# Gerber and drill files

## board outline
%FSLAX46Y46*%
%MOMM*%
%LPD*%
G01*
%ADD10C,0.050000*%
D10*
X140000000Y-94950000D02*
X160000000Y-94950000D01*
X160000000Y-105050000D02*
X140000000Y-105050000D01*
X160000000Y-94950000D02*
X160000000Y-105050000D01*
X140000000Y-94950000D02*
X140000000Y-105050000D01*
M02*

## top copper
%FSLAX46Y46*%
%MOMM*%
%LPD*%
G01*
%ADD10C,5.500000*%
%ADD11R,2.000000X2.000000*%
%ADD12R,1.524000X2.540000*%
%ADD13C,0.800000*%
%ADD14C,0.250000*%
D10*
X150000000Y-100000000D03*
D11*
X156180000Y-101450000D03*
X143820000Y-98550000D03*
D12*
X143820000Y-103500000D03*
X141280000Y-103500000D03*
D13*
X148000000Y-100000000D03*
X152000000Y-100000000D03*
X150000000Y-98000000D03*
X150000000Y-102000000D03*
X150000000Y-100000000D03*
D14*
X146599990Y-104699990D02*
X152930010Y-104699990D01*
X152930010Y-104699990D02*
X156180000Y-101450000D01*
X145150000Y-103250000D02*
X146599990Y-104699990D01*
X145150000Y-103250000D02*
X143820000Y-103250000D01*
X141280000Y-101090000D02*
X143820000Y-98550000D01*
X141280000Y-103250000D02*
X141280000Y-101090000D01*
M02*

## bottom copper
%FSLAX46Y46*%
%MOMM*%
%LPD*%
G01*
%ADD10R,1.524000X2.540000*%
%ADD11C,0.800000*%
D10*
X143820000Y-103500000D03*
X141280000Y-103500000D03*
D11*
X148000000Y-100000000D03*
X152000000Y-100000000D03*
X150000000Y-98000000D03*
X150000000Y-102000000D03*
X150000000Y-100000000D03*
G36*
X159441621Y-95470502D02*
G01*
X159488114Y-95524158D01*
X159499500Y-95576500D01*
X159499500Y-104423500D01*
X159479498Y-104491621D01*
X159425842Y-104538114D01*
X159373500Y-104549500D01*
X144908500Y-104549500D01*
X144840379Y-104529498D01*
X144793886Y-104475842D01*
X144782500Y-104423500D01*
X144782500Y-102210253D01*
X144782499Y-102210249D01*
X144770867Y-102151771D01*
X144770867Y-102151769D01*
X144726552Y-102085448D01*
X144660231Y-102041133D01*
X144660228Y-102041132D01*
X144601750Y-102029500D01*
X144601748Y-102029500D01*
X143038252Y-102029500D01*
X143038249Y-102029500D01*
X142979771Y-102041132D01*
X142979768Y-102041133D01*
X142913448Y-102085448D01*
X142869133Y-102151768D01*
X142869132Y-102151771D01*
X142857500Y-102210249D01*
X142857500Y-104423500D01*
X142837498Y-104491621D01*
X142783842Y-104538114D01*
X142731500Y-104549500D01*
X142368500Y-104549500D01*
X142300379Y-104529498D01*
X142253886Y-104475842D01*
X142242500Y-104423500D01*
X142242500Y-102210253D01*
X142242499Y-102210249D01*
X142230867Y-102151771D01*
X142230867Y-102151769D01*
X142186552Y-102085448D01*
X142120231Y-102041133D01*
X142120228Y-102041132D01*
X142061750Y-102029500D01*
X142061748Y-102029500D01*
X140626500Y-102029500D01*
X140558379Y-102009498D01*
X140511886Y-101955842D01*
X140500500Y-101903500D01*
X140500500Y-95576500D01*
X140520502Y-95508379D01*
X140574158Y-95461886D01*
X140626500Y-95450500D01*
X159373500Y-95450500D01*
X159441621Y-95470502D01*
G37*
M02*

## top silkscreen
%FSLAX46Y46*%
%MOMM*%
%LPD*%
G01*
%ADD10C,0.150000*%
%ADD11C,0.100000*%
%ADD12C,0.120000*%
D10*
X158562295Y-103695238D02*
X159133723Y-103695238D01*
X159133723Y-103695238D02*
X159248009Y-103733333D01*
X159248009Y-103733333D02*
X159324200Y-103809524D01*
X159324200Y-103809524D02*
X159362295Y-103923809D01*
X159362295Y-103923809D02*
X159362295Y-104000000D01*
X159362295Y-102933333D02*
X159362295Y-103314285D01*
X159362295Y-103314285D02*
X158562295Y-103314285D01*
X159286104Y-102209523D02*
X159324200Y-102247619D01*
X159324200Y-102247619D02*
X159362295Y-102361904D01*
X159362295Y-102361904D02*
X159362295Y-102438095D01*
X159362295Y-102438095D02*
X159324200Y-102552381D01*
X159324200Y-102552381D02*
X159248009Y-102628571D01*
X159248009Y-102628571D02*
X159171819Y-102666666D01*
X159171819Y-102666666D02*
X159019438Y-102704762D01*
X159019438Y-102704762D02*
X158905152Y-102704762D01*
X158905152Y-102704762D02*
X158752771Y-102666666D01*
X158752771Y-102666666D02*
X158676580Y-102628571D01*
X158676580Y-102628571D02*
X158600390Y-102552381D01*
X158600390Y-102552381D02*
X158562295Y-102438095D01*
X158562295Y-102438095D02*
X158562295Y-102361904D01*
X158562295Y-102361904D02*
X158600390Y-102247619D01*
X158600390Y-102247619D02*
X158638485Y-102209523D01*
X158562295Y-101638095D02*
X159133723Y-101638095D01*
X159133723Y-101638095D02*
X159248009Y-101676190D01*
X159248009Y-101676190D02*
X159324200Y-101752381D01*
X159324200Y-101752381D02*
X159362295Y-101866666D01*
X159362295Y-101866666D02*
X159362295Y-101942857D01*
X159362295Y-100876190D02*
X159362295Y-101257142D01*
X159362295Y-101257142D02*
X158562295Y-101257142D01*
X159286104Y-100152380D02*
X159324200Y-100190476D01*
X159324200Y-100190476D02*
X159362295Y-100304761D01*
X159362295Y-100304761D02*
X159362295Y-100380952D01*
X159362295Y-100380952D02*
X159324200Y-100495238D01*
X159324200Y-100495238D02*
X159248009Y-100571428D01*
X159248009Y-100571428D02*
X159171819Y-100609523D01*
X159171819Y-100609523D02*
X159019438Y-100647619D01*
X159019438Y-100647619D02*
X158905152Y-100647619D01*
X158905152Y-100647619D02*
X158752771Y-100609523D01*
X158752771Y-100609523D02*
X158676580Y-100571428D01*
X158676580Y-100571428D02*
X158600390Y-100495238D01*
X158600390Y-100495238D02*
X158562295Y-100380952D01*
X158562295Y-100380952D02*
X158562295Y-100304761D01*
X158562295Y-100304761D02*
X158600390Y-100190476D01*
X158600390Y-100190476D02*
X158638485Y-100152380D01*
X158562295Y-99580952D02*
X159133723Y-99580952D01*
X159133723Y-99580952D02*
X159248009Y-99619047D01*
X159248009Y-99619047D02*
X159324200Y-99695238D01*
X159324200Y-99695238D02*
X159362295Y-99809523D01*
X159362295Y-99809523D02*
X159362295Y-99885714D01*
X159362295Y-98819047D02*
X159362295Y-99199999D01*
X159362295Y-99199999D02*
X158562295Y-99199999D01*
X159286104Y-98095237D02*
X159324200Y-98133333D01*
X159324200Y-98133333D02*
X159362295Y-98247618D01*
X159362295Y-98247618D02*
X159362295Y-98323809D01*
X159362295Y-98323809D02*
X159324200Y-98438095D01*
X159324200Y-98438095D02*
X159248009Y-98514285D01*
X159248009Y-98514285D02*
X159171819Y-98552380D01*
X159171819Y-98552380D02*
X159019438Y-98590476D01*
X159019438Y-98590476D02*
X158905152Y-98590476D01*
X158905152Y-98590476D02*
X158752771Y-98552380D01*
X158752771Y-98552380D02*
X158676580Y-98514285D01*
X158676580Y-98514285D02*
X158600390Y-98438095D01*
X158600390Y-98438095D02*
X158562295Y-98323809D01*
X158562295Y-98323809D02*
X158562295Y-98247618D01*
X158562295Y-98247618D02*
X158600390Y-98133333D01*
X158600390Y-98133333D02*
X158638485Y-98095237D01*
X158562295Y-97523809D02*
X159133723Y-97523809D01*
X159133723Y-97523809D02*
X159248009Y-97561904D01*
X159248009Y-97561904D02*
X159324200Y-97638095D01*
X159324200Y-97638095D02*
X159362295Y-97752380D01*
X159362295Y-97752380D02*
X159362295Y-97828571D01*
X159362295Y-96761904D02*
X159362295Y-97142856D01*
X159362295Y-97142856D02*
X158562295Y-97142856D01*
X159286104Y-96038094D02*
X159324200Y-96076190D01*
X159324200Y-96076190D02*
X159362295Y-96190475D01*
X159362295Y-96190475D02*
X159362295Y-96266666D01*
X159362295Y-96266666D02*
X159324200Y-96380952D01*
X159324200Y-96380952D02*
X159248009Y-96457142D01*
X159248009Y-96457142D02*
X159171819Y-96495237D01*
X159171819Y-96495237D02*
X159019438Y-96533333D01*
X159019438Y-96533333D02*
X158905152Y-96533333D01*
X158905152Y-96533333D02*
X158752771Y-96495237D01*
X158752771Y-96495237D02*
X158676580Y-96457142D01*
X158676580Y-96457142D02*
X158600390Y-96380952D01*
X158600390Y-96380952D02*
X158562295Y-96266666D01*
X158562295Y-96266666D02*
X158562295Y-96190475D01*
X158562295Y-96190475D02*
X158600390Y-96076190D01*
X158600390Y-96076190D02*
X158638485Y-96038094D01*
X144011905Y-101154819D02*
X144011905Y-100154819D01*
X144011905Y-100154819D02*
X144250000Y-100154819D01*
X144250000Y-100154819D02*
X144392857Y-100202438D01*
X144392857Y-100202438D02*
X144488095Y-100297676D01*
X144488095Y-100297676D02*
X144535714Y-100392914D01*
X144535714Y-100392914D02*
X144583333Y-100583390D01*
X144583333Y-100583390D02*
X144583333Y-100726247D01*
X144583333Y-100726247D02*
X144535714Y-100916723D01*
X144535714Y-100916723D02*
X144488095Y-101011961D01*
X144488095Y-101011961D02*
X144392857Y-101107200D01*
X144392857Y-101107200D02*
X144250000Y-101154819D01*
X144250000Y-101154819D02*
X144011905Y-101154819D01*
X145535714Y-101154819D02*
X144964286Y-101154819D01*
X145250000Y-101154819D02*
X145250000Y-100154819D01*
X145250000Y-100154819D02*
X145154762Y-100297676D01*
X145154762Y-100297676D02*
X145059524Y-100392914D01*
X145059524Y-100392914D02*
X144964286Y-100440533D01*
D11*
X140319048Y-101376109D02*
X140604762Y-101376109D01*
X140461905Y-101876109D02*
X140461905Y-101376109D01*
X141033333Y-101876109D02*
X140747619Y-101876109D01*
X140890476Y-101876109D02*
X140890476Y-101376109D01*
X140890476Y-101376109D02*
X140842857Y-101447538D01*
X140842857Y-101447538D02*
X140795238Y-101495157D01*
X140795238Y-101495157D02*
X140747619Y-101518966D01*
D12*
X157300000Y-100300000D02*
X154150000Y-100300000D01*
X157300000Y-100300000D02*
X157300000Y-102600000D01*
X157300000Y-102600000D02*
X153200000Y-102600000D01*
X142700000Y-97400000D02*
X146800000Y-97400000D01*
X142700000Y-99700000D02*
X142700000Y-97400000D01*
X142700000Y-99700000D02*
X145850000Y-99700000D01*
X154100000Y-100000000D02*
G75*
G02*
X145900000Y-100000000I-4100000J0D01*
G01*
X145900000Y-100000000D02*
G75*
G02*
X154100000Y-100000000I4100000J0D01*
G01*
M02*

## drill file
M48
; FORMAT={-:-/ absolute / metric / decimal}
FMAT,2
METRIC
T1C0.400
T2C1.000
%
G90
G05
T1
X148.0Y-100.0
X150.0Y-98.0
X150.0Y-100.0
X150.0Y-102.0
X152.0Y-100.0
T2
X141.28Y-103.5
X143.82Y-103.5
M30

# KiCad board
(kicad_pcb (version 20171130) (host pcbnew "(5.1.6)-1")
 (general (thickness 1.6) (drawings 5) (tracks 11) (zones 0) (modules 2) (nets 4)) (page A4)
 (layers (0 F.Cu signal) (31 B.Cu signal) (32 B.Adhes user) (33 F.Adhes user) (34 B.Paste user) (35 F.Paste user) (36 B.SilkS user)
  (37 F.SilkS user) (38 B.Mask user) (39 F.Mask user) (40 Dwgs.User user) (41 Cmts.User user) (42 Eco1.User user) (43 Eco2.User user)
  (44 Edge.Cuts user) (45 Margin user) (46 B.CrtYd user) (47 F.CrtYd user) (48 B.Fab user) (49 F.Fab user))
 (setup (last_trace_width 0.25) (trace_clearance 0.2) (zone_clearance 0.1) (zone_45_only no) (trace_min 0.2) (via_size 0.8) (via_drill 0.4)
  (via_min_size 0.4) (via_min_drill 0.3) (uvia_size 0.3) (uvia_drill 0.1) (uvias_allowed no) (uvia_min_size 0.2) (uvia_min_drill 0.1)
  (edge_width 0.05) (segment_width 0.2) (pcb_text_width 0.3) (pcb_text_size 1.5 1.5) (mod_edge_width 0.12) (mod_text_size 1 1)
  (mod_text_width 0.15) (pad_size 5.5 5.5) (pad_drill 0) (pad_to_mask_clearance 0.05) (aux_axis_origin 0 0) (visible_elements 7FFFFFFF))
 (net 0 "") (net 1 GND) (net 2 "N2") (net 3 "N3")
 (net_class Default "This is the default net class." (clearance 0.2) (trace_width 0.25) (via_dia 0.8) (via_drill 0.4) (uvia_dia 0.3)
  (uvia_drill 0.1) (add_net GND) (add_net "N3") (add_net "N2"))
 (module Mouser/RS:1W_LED (layer F.Cu) (at 150 100)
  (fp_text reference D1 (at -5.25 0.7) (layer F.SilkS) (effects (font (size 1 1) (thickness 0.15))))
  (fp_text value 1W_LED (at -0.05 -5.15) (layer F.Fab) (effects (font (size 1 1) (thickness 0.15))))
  (fp_line (start 7.3 0.3) (end 4.15 0.3) (layer F.SilkS) (width 0.12))
  (fp_line (start 7.3 0.3) (end 7.3 2.6) (layer F.SilkS) (width 0.12))
  (fp_line (start 7.3 2.6) (end 3.2 2.6) (layer F.SilkS) (width 0.12))
  (fp_line (start -7.3 -2.6) (end -3.2 -2.6) (layer F.SilkS) (width 0.12))
  (fp_line (start -7.3 -0.3) (end -7.3 -2.6) (layer F.SilkS) (width 0.12))
  (fp_line (start -7.3 -0.3) (end -4.15 -0.3) (layer F.SilkS) (width 0.12))
  (fp_circle (center 0 0) (end 4.1 0) (layer F.SilkS) (width 0.12))
  (pad 3 smd circle (at 0 0) (size 5.5 5.5) (layers F.Cu F.Paste F.Mask) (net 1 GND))
  (pad 2 smd rect (at 6.18 1.45) (size 2 2) (layers F.Cu F.Paste F.Mask) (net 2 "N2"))
  (pad 1 smd rect (at -6.18 -1.45) (size 2 2) (layers F.Cu F.Paste F.Mask) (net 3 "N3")))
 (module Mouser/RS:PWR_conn (layer F.Cu) (at 142.55 103.5 180)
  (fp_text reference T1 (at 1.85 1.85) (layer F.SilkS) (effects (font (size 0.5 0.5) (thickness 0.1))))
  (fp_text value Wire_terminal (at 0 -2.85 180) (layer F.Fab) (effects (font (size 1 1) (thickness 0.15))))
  (pad 2 thru_hole rect (at -1.27 0 180) (size 1.524 2.54) (drill 1) (layers *.Cu *.Mask) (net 2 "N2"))
  (pad 1 thru_hole rect (at 1.27 0 180) (size 1.524 2.54) (drill 1) (layers *.Cu *.Mask) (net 3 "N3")))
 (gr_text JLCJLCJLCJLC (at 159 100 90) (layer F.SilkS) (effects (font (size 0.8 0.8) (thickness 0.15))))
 (gr_line (start 140 94.95) (end 160 94.95) (layer Edge.Cuts) (width 0.05))
 (gr_line (start 160 105.05) (end 140 105.05) (layer Edge.Cuts) (width 0.05))
 (gr_line (start 160 94.95) (end 160 105.05) (layer Edge.Cuts) (width 0.05))
 (gr_line (start 140 94.95) (end 140 105.05) (layer Edge.Cuts) (width 0.05))
 (segment (start 146.59999 104.69999) (end 152.93001 104.69999) (width 0.25) (layer F.Cu) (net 2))
 (segment (start 152.93001 104.69999) (end 156.18 101.45) (width 0.25) (layer F.Cu) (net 2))
 (segment (start 145.15 103.25) (end 146.59999 104.69999) (width 0.25) (layer F.Cu) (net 2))
 (segment (start 145.15 103.25) (end 143.82 103.25) (width 0.25) (layer F.Cu) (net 2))
 (segment (start 141.28 101.09) (end 143.82 98.55) (width 0.25) (layer F.Cu) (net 3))
 (segment (start 141.28 103.25) (end 141.28 101.09) (width 0.25) (layer F.Cu) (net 3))
 (via (at 148 100) (size 0.8) (drill 0.4) (layers F.Cu B.Cu) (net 1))
 (via (at 152 100) (size 0.8) (drill 0.4) (layers F.Cu B.Cu) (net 1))
 (via (at 150 98) (size 0.8) (drill 0.4) (layers F.Cu B.Cu) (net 1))
 (via (at 150 102) (size 0.8) (drill 0.4) (layers F.Cu B.Cu) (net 1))
 (via (at 150 100) (size 0.8) (drill 0.4) (layers F.Cu B.Cu) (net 1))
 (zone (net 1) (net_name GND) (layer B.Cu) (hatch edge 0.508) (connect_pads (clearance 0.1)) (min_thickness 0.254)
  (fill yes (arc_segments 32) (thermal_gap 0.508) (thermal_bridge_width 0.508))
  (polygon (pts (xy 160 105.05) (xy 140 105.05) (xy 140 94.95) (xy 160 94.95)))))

